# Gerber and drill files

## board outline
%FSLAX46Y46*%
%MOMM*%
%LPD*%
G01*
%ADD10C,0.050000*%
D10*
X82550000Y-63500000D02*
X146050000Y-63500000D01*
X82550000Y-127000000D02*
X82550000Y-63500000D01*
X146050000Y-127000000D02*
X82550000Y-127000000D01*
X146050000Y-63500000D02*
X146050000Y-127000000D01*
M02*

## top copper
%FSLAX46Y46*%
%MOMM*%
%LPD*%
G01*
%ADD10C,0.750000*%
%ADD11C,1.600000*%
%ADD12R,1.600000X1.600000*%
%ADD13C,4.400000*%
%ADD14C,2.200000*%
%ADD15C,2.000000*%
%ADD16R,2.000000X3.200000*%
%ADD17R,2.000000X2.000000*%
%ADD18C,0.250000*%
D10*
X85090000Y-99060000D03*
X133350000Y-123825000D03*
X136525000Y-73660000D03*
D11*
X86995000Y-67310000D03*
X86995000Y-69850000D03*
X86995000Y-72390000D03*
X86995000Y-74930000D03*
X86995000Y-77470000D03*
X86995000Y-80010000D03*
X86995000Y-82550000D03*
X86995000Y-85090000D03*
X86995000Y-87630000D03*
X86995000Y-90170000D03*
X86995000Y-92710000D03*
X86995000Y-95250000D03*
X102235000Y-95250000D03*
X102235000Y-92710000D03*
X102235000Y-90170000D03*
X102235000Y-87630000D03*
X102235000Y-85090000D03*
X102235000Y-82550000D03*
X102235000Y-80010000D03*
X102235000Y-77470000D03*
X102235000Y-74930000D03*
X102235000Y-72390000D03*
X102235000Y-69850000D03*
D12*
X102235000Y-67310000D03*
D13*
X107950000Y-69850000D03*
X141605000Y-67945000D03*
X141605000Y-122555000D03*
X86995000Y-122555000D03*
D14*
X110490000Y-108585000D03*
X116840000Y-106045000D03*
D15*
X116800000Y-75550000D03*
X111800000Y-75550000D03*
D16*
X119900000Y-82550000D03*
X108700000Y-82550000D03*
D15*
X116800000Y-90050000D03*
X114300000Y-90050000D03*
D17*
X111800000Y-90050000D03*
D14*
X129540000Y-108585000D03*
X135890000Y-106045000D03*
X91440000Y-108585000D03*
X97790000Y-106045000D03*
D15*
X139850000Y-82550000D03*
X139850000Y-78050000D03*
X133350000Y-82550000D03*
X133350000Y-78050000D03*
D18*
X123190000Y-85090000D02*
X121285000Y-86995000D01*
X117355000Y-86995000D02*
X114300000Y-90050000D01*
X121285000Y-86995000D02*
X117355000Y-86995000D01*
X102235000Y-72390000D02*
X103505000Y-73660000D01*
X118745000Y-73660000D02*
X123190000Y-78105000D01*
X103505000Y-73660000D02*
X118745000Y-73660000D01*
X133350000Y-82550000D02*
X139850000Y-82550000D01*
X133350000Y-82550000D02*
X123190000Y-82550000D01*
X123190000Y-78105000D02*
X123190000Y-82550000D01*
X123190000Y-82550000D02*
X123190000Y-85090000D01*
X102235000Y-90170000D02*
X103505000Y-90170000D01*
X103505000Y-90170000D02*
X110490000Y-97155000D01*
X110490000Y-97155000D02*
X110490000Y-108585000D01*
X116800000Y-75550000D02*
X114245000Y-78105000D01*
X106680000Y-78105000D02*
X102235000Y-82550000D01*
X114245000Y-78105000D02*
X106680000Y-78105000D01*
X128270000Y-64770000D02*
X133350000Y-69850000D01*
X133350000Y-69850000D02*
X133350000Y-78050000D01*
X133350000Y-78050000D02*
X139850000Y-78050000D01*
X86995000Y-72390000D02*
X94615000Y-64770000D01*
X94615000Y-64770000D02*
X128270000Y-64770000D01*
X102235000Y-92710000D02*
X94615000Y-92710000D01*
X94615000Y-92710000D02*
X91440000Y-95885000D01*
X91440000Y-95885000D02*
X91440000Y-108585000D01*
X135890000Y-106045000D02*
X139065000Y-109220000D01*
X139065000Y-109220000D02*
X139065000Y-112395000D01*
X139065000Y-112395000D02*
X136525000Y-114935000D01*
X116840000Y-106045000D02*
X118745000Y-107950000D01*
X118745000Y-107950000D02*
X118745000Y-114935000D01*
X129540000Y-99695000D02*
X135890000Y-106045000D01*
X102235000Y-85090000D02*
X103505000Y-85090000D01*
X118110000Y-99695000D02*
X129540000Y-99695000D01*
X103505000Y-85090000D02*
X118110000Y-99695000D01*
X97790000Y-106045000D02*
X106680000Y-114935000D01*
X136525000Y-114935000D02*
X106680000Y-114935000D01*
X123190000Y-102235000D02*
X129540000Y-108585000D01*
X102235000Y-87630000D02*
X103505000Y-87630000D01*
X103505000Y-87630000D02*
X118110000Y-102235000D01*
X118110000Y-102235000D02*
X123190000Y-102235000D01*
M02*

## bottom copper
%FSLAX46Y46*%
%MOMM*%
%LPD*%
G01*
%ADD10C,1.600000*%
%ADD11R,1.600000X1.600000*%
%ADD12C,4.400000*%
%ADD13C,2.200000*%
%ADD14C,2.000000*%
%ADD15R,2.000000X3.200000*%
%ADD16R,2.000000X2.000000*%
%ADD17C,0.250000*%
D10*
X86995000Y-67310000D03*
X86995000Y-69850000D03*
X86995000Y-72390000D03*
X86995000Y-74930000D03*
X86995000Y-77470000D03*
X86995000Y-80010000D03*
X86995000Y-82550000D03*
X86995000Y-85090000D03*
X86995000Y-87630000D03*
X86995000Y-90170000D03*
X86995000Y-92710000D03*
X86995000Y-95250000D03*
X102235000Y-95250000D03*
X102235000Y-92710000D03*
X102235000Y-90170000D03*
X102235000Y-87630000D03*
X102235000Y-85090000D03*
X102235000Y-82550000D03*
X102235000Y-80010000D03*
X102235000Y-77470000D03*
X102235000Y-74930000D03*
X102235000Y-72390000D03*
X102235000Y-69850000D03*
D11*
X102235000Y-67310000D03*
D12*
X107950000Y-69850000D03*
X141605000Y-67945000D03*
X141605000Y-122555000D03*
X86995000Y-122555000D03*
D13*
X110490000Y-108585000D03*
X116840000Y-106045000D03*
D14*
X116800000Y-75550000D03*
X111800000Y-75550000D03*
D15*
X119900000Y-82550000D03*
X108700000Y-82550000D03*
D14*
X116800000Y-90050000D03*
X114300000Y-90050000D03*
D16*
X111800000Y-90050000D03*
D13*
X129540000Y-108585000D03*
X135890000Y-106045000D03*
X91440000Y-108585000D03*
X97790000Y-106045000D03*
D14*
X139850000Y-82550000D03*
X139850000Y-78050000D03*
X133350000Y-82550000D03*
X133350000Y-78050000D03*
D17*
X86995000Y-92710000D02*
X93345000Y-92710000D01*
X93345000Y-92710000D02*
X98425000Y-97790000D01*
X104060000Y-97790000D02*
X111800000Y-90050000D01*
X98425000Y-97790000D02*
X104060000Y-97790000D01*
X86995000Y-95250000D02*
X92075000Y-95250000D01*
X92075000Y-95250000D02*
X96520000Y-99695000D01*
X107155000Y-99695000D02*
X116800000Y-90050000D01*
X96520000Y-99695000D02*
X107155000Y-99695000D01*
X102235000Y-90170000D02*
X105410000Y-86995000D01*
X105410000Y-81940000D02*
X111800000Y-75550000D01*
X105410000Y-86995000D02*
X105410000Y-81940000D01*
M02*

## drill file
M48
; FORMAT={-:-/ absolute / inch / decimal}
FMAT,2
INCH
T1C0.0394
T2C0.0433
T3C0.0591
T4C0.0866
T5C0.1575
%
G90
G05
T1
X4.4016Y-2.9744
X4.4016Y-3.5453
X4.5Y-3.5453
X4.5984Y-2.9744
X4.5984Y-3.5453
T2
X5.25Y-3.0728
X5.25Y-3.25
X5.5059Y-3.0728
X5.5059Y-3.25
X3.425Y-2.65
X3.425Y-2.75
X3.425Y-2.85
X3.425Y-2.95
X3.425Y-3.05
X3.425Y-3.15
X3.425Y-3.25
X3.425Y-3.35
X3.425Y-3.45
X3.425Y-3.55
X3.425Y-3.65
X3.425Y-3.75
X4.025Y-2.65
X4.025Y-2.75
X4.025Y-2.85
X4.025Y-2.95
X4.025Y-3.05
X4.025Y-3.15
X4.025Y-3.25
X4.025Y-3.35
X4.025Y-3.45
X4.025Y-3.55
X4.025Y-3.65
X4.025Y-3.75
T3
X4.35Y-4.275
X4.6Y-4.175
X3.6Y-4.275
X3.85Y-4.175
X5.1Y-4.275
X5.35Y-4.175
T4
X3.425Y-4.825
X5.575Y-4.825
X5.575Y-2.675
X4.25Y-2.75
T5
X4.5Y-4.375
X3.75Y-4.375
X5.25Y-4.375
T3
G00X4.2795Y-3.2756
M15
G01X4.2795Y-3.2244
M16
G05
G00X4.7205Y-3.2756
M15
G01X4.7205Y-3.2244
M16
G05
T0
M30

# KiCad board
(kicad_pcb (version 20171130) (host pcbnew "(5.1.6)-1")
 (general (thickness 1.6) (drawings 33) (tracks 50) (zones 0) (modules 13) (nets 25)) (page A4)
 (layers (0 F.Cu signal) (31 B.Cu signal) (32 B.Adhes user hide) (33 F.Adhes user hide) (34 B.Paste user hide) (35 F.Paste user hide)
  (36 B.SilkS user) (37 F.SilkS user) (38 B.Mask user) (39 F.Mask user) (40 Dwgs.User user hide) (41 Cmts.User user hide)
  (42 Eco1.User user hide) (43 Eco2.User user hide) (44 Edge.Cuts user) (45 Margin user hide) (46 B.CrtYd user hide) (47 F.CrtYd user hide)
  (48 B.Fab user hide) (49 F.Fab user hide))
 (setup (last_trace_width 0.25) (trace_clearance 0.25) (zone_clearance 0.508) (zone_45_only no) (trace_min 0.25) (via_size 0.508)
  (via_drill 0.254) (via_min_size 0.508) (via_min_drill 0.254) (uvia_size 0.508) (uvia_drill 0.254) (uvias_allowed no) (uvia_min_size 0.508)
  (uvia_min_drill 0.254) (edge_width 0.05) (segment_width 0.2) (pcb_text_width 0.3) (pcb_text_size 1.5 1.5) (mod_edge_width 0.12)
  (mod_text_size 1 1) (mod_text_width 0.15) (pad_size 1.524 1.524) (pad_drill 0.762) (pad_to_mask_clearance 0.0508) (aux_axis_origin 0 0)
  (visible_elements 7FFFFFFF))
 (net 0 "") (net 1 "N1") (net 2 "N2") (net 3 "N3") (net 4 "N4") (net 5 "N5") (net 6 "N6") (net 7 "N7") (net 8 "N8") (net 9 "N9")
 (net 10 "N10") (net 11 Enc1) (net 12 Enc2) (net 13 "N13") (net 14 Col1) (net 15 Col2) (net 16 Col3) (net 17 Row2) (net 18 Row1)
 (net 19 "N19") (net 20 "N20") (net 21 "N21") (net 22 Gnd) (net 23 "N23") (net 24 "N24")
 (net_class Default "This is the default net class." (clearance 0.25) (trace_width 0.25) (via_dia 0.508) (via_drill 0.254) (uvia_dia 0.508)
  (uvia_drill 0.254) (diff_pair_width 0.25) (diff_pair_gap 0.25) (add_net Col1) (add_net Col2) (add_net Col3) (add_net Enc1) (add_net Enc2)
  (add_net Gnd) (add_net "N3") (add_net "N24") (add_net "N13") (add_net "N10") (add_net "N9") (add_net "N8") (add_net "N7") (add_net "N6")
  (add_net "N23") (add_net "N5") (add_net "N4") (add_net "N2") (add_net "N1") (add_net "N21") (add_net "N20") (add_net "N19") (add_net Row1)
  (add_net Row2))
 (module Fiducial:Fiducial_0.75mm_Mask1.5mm (layer F.Cu) (at 85.09 99.06)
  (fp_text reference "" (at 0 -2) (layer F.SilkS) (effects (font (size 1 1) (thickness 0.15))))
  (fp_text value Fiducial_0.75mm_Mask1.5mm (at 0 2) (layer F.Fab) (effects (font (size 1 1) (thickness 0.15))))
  (pad "" smd circle (at 0 0) (size 0.75 0.75) (layers F.Cu F.Mask) (solder_mask_margin 0.375) (clearance 0.375)))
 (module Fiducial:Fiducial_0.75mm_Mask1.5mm (layer F.Cu) (at 133.35 123.825)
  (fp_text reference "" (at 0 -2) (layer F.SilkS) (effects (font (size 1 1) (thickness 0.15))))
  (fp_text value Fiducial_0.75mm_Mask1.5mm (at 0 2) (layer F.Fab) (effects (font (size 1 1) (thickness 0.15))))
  (pad "" smd circle (at 0 0) (size 0.75 0.75) (layers F.Cu F.Mask) (solder_mask_margin 0.375) (clearance 0.375)))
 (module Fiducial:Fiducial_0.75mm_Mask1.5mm (layer F.Cu) (at 136.525 73.66)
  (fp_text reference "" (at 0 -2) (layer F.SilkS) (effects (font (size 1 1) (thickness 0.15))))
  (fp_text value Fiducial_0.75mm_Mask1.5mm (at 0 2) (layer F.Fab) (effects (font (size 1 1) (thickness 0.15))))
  (pad "" smd circle (at 0 0) (size 0.75 0.75) (layers F.Cu F.Mask) (solder_mask_margin 0.375) (clearance 0.375)))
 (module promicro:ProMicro (layer B.Cu) (at 94.615 81.28 270)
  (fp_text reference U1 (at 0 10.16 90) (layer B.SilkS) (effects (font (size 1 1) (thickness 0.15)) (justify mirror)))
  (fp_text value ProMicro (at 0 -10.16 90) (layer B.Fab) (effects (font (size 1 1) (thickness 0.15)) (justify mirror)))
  (pad 24 thru_hole circle (at -13.97 7.62 270) (size 1.6 1.6) (drill 1.1) (layers *.Cu *.Mask B.SilkS) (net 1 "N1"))
  (pad 23 thru_hole circle (at -11.43 7.62 270) (size 1.6 1.6) (drill 1.1) (layers *.Cu *.Mask B.SilkS) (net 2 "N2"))
  (pad 22 thru_hole circle (at -8.89 7.62 270) (size 1.6 1.6) (drill 1.1) (layers *.Cu *.Mask B.SilkS) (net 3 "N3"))
  (pad 21 thru_hole circle (at -6.35 7.62 270) (size 1.6 1.6) (drill 1.1) (layers *.Cu *.Mask B.SilkS) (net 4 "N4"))
  (pad 20 thru_hole circle (at -3.81 7.62 270) (size 1.6 1.6) (drill 1.1) (layers *.Cu *.Mask B.SilkS) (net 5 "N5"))
  (pad 19 thru_hole circle (at -1.27 7.62 270) (size 1.6 1.6) (drill 1.1) (layers *.Cu *.Mask B.SilkS) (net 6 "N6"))
  (pad 18 thru_hole circle (at 1.27 7.62 270) (size 1.6 1.6) (drill 1.1) (layers *.Cu *.Mask B.SilkS) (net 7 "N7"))
  (pad 17 thru_hole circle (at 3.81 7.62 270) (size 1.6 1.6) (drill 1.1) (layers *.Cu *.Mask B.SilkS) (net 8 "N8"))
  (pad 16 thru_hole circle (at 6.35 7.62 270) (size 1.6 1.6) (drill 1.1) (layers *.Cu *.Mask B.SilkS) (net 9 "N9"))
  (pad 15 thru_hole circle (at 8.89 7.62 270) (size 1.6 1.6) (drill 1.1) (layers *.Cu *.Mask B.SilkS) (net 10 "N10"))
  (pad 14 thru_hole circle (at 11.43 7.62 270) (size 1.6 1.6) (drill 1.1) (layers *.Cu *.Mask B.SilkS) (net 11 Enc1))
  (pad 13 thru_hole circle (at 13.97 7.62 270) (size 1.6 1.6) (drill 1.1) (layers *.Cu *.Mask B.SilkS) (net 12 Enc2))
  (pad 12 thru_hole circle (at 13.97 -7.62 270) (size 1.6 1.6) (drill 1.1) (layers *.Cu *.Mask B.SilkS) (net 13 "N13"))
  (pad 11 thru_hole circle (at 11.43 -7.62 270) (size 1.6 1.6) (drill 1.1) (layers *.Cu *.Mask B.SilkS) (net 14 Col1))
  (pad 10 thru_hole circle (at 8.89 -7.62 270) (size 1.6 1.6) (drill 1.1) (layers *.Cu *.Mask B.SilkS) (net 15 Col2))
  (pad 9 thru_hole circle (at 6.35 -7.62 270) (size 1.6 1.6) (drill 1.1) (layers *.Cu *.Mask B.SilkS) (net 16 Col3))
  (pad 8 thru_hole circle (at 3.81 -7.62 270) (size 1.6 1.6) (drill 1.1) (layers *.Cu *.Mask B.SilkS) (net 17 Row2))
  (pad 7 thru_hole circle (at 1.27 -7.62 270) (size 1.6 1.6) (drill 1.1) (layers *.Cu *.Mask B.SilkS) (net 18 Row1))
  (pad 6 thru_hole circle (at -1.27 -7.62 270) (size 1.6 1.6) (drill 1.1) (layers *.Cu *.Mask B.SilkS) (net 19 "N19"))
  (pad 5 thru_hole circle (at -3.81 -7.62 270) (size 1.6 1.6) (drill 1.1) (layers *.Cu *.Mask B.SilkS) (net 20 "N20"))
  (pad 4 thru_hole circle (at -6.35 -7.62 270) (size 1.6 1.6) (drill 1.1) (layers *.Cu *.Mask B.SilkS) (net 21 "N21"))
  (pad 3 thru_hole circle (at -8.89 -7.62 270) (size 1.6 1.6) (drill 1.1) (layers *.Cu *.Mask B.SilkS) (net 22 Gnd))
  (pad 2 thru_hole circle (at -11.43 -7.62 270) (size 1.6 1.6) (drill 1.1) (layers *.Cu *.Mask B.SilkS) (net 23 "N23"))
  (pad 1 thru_hole rect (at -13.97 -7.62 270) (size 1.6 1.6) (drill 1.1) (layers *.Cu *.Mask B.SilkS) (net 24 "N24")))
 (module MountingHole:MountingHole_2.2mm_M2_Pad (layer F.Cu) (at 107.95 69.85)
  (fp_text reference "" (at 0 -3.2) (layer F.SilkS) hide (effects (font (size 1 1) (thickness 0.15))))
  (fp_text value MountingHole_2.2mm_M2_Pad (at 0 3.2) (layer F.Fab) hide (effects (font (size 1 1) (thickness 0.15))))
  (pad 1 thru_hole circle (at 0 0) (size 4.4 4.4) (drill 2.2) (layers *.Cu *.Mask)))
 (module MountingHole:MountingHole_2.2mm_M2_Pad (layer F.Cu) (at 141.605 67.945)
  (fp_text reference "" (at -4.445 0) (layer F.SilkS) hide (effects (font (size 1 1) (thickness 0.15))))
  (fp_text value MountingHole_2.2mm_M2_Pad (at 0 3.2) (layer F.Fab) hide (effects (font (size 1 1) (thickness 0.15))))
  (pad 1 thru_hole circle (at 0 0) (size 4.4 4.4) (drill 2.2) (layers *.Cu *.Mask)))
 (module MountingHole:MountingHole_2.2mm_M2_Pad (layer F.Cu) (at 141.605 122.555)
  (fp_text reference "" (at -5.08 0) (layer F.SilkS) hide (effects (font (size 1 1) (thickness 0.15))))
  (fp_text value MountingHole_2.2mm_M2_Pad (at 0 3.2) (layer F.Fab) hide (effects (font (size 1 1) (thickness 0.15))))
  (pad 1 thru_hole circle (at 0 0) (size 4.4 4.4) (drill 2.2) (layers *.Cu *.Mask)))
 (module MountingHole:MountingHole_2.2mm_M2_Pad (layer F.Cu) (at 86.995 122.555)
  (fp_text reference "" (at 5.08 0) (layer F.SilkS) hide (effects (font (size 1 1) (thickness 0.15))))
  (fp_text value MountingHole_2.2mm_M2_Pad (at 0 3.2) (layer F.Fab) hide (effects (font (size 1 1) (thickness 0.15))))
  (pad 1 thru_hole circle (at 0 0) (size 4.4 4.4) (drill 2.2) (layers *.Cu *.Mask)))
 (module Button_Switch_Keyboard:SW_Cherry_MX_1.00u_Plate (layer F.Cu) (at 116.84 106.045)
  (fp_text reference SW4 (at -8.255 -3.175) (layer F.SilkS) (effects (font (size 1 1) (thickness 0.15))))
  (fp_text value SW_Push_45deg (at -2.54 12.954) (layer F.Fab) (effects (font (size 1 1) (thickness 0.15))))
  (pad "" np_thru_hole circle (at -2.54 5.08) (size 4 4) (drill 4) (layers *.Cu *.Mask))
  (pad 2 thru_hole circle (at -6.35 2.54) (size 2.2 2.2) (drill 1.5) (layers *.Cu *.Mask) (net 15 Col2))
  (pad 1 thru_hole circle (at 0 0) (size 2.2 2.2) (drill 1.5) (layers *.Cu *.Mask) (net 17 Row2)))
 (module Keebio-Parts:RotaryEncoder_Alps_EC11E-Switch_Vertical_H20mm (layer F.Cu) (at 114.3 82.55 90)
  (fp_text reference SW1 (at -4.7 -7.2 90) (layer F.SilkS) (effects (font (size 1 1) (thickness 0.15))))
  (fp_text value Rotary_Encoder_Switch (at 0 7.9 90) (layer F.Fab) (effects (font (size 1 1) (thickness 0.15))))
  (pad S1 thru_hole circle (at 7 2.5 90) (size 2 2) (drill 1) (layers *.Cu *.Mask) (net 18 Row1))
  (pad S2 thru_hole circle (at 7 -2.5 90) (size 2 2) (drill 1) (layers *.Cu *.Mask) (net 15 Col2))
  (pad MP thru_hole rect (at 0 5.6 90) (size 3.2 2) (drill oval 2.8 1.5) (layers *.Cu *.Mask))
  (pad MP thru_hole rect (at 0 -5.6 90) (size 3.2 2) (drill oval 2.8 1.5) (layers *.Cu *.Mask))
  (pad B thru_hole circle (at -7.5 2.5 90) (size 2 2) (drill 1) (layers *.Cu *.Mask) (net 12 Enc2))
  (pad C thru_hole circle (at -7.5 0 90) (size 2 2) (drill 1) (layers *.Cu *.Mask) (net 22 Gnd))
  (pad A thru_hole rect (at -7.5 -2.5 90) (size 2 2) (drill 1) (layers *.Cu *.Mask) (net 11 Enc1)))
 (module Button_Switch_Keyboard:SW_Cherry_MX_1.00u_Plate (layer F.Cu) (at 135.89 106.045)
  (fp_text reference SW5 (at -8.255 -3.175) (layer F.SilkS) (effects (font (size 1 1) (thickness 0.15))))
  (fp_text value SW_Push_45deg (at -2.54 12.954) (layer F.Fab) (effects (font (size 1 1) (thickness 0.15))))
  (pad "" np_thru_hole circle (at -2.54 5.08) (size 4 4) (drill 4) (layers *.Cu *.Mask))
  (pad 2 thru_hole circle (at -6.35 2.54) (size 2.2 2.2) (drill 1.5) (layers *.Cu *.Mask) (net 16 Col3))
  (pad 1 thru_hole circle (at 0 0) (size 2.2 2.2) (drill 1.5) (layers *.Cu *.Mask) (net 17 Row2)))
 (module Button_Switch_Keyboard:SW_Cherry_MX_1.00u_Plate (layer F.Cu) (at 97.79 106.045)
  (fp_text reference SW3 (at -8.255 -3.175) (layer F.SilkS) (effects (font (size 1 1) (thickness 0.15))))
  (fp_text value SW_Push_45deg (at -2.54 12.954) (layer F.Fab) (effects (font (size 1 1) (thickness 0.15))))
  (pad "" np_thru_hole circle (at -2.54 5.08) (size 4 4) (drill 4) (layers *.Cu *.Mask))
  (pad 2 thru_hole circle (at -6.35 2.54) (size 2.2 2.2) (drill 1.5) (layers *.Cu *.Mask) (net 14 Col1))
  (pad 1 thru_hole circle (at 0 0) (size 2.2 2.2) (drill 1.5) (layers *.Cu *.Mask) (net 17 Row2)))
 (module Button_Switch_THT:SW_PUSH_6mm (layer B.Cu) (at 133.35 82.55)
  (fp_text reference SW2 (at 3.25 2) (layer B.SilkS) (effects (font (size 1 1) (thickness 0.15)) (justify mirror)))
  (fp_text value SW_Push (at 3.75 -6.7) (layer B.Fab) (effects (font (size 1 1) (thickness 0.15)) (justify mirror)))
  (pad 1 thru_hole circle (at 6.5 0 270) (size 2 2) (drill 1.1) (layers *.Cu *.Mask) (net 22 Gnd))
  (pad 2 thru_hole circle (at 6.5 -4.5 270) (size 2 2) (drill 1.1) (layers *.Cu *.Mask) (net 3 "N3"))
  (pad 1 thru_hole circle (at 0 0 270) (size 2 2) (drill 1.1) (layers *.Cu *.Mask) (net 22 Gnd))
  (pad 2 thru_hole circle (at 0 -4.5 270) (size 2 2) (drill 1.1) (layers *.Cu *.Mask) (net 3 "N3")))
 (gr_line (start 82.55 63.5) (end 146.05 63.5) (layer Edge.Cuts) (width 0.05))
 (gr_line (start 82.55 127) (end 82.55 63.5) (layer Edge.Cuts) (width 0.05))
 (gr_line (start 146.05 127) (end 82.55 127) (layer Edge.Cuts) (width 0.05))
 (gr_line (start 146.05 63.5) (end 146.05 127) (layer Edge.Cuts) (width 0.05))
 (segment (start 86.995 92.71) (end 93.345 92.71) (width 0.25) (layer B.Cu) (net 11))
 (segment (start 93.345 92.71) (end 98.425 97.79) (width 0.25) (layer B.Cu) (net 11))
 (segment (start 104.06 97.79) (end 111.8 90.05) (width 0.25) (layer B.Cu) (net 11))
 (segment (start 98.425 97.79) (end 104.06 97.79) (width 0.25) (layer B.Cu) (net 11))
 (segment (start 123.19 85.09) (end 121.285 86.995) (width 0.25) (layer F.Cu) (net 22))
 (segment (start 117.355 86.995) (end 114.3 90.05) (width 0.25) (layer F.Cu) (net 22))
 (segment (start 121.285 86.995) (end 117.355 86.995) (width 0.25) (layer F.Cu) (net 22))
 (segment (start 102.235 72.39) (end 103.505 73.66) (width 0.25) (layer F.Cu) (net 22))
 (segment (start 118.745 73.66) (end 123.19 78.105) (width 0.25) (layer F.Cu) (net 22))
 (segment (start 103.505 73.66) (end 118.745 73.66) (width 0.25) (layer F.Cu) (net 22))
 (segment (start 133.35 82.55) (end 139.85 82.55) (width 0.25) (layer F.Cu) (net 22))
 (segment (start 133.35 82.55) (end 123.19 82.55) (width 0.25) (layer F.Cu) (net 22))
 (segment (start 123.19 78.105) (end 123.19 82.55) (width 0.25) (layer F.Cu) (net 22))
 (segment (start 123.19 82.55) (end 123.19 85.09) (width 0.25) (layer F.Cu) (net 22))
 (segment (start 86.995 95.25) (end 92.075 95.25) (width 0.25) (layer B.Cu) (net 12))
 (segment (start 92.075 95.25) (end 96.52 99.695) (width 0.25) (layer B.Cu) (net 12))
 (segment (start 107.155 99.695) (end 116.8 90.05) (width 0.25) (layer B.Cu) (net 12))
 (segment (start 96.52 99.695) (end 107.155 99.695) (width 0.25) (layer B.Cu) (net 12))
 (segment (start 102.235 90.17) (end 105.41 86.995) (width 0.25) (layer B.Cu) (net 15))
 (segment (start 105.41 81.94) (end 111.8 75.55) (width 0.25) (layer B.Cu) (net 15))
 (segment (start 105.41 86.995) (end 105.41 81.94) (width 0.25) (layer B.Cu) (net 15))
 (segment (start 102.235 90.17) (end 103.505 90.17) (width 0.25) (layer F.Cu) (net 15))
 (segment (start 103.505 90.17) (end 110.49 97.155) (width 0.25) (layer F.Cu) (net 15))
 (segment (start 110.49 97.155) (end 110.49 108.585) (width 0.25) (layer F.Cu) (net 15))
 (segment (start 116.8 75.55) (end 114.245 78.105) (width 0.25) (layer F.Cu) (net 18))
 (segment (start 106.68 78.105) (end 102.235 82.55) (width 0.25) (layer F.Cu) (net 18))
 (segment (start 114.245 78.105) (end 106.68 78.105) (width 0.25) (layer F.Cu) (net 18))
 (segment (start 128.27 64.77) (end 133.35 69.85) (width 0.25) (layer F.Cu) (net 3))
 (segment (start 133.35 69.85) (end 133.35 78.05) (width 0.25) (layer F.Cu) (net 3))
 (segment (start 133.35 78.05) (end 139.85 78.05) (width 0.25) (layer F.Cu) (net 3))
 (segment (start 86.995 72.39) (end 94.615 64.77) (width 0.25) (layer F.Cu) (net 3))
 (segment (start 94.615 64.77) (end 128.27 64.77) (width 0.25) (layer F.Cu) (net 3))
 (segment (start 102.235 92.71) (end 94.615 92.71) (width 0.25) (layer F.Cu) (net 14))
 (segment (start 94.615 92.71) (end 91.44 95.885) (width 0.25) (layer F.Cu) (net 14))
 (segment (start 91.44 95.885) (end 91.44 108.585) (width 0.25) (layer F.Cu) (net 14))
 (segment (start 135.89 106.045) (end 139.065 109.22) (width 0.25) (layer F.Cu) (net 17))
 (segment (start 139.065 109.22) (end 139.065 112.395) (width 0.25) (layer F.Cu) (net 17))
 (segment (start 139.065 112.395) (end 136.525 114.935) (width 0.25) (layer F.Cu) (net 17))
 (segment (start 116.84 106.045) (end 118.745 107.95) (width 0.25) (layer F.Cu) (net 17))
 (segment (start 118.745 107.95) (end 118.745 114.935) (width 0.25) (layer F.Cu) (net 17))
 (segment (start 129.54 99.695) (end 135.89 106.045) (width 0.25) (layer F.Cu) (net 17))
 (segment (start 102.235 85.09) (end 103.505 85.09) (width 0.25) (layer F.Cu) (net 17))
 (segment (start 118.11 99.695) (end 129.54 99.695) (width 0.25) (layer F.Cu) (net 17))
 (segment (start 103.505 85.09) (end 118.11 99.695) (width 0.25) (layer F.Cu) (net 17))
 (segment (start 97.79 106.045) (end 106.68 114.935) (width 0.25) (layer F.Cu) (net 17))
 (segment (start 136.525 114.935) (end 106.68 114.935) (width 0.25) (layer F.Cu) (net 17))
 (segment (start 123.19 102.235) (end 129.54 108.585) (width 0.25) (layer F.Cu) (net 16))
 (segment (start 102.235 87.63) (end 103.505 87.63) (width 0.25) (layer F.Cu) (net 16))
 (segment (start 103.505 87.63) (end 118.11 102.235) (width 0.25) (layer F.Cu) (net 16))
 (segment (start 118.11 102.235) (end 123.19 102.235) (width 0.25) (layer F.Cu) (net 16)))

